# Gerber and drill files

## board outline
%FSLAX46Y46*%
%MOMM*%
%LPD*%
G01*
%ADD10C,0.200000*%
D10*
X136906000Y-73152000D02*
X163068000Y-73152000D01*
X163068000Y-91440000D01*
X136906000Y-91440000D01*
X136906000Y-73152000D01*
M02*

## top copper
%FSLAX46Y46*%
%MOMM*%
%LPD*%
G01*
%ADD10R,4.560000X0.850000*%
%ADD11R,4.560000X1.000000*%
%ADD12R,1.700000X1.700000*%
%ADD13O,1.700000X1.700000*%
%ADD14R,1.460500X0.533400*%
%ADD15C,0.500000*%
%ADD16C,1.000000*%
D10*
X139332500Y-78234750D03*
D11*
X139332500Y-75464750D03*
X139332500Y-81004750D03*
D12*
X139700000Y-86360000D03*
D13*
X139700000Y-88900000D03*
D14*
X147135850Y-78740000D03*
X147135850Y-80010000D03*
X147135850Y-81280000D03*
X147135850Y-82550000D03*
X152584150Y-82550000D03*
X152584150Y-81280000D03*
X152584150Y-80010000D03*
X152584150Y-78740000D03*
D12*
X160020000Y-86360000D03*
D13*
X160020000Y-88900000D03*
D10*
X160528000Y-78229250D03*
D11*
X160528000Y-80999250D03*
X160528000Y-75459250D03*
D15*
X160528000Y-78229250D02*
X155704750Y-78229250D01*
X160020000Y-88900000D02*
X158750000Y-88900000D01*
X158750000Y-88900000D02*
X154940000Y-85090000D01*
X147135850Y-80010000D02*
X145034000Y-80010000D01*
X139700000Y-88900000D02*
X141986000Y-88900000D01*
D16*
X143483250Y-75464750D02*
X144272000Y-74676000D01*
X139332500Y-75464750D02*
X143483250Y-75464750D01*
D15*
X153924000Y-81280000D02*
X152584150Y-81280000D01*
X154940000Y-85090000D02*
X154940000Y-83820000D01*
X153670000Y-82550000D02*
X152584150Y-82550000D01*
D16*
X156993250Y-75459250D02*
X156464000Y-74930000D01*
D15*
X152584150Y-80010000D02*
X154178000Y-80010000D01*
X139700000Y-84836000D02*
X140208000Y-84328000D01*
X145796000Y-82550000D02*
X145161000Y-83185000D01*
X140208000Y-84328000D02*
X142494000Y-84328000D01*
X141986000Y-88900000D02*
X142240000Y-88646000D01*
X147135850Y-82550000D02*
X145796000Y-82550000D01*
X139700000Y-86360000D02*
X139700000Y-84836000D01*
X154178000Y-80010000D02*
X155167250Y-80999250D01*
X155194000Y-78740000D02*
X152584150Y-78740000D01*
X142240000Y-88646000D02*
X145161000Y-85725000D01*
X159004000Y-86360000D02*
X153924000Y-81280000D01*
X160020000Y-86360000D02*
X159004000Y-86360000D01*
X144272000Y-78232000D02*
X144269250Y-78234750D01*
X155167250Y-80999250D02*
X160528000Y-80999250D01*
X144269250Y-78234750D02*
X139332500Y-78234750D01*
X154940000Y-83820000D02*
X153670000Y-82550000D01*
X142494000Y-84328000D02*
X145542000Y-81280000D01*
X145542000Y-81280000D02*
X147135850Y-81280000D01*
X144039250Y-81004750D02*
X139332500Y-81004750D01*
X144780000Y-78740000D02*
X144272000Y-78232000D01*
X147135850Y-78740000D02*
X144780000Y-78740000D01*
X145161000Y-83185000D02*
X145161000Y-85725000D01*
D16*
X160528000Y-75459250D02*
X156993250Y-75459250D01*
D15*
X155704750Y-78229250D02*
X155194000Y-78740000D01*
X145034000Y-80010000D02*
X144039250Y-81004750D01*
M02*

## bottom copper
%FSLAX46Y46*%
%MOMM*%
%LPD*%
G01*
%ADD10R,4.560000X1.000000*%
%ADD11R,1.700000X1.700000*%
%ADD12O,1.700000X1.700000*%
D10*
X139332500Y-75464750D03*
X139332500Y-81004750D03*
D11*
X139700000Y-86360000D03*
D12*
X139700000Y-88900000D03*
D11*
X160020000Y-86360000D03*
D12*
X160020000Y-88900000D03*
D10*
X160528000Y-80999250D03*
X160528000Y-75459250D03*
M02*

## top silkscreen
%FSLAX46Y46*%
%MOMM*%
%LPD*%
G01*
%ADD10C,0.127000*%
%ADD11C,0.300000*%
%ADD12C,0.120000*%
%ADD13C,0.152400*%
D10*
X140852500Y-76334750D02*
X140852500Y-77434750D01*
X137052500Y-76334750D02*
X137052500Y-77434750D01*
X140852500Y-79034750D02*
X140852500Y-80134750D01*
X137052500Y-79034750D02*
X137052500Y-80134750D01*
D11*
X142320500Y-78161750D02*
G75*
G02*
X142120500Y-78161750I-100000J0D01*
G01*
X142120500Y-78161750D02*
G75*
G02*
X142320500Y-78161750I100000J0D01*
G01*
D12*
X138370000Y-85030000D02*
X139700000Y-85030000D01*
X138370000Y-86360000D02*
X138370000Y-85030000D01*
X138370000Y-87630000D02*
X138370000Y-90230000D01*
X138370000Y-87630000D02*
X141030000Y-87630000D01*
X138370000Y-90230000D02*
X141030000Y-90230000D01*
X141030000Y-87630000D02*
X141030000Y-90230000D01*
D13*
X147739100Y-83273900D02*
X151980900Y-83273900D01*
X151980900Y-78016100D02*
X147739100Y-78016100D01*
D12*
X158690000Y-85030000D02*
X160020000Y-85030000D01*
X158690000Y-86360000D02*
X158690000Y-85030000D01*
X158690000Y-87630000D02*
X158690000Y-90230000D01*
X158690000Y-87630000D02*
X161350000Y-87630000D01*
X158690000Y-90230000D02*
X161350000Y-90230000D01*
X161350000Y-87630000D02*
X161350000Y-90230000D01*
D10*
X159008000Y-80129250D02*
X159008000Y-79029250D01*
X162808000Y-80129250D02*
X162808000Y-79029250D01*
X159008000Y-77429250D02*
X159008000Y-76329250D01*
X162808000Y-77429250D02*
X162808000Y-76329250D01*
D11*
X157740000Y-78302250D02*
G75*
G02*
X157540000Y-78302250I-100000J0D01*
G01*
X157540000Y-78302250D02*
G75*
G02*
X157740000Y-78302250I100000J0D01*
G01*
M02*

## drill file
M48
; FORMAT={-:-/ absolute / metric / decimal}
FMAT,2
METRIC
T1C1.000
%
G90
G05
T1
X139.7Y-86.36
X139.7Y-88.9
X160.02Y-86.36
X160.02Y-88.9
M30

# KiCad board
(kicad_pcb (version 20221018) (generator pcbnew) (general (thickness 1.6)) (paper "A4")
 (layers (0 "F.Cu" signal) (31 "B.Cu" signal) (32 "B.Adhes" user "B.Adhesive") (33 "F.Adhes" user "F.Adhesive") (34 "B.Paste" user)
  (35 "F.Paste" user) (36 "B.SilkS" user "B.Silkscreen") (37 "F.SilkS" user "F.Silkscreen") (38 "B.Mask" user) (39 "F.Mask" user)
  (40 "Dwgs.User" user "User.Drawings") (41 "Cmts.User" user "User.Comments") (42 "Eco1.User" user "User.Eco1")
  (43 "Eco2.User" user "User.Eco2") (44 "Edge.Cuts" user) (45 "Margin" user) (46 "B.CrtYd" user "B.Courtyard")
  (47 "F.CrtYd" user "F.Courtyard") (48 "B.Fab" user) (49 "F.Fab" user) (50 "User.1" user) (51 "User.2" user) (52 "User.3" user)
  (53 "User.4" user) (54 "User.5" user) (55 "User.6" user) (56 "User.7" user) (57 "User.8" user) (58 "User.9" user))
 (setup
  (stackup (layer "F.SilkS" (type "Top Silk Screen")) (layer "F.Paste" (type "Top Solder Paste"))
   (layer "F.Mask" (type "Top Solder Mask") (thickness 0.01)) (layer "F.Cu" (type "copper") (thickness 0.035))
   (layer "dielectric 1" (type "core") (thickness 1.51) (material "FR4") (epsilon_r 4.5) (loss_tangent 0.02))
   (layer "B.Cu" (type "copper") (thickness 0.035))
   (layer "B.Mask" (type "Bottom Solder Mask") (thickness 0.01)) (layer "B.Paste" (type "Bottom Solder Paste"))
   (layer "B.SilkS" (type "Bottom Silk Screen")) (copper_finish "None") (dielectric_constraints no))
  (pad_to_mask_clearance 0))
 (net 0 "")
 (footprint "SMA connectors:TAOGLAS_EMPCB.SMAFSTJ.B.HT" (layer "F.Cu") (at 139.3325 78.23475 -90)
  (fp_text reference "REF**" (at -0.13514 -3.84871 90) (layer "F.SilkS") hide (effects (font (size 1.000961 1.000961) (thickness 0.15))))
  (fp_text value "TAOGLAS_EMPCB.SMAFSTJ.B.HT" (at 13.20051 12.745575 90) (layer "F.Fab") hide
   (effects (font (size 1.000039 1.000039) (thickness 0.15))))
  (fp_line (start -1.9 -1.52) (end -0.8 -1.52) (stroke (width 0.127) (type solid)) (layer "F.SilkS"))
  (fp_line (start -1.9 2.28) (end -0.8 2.28) (stroke (width 0.127) (type solid)) (layer "F.SilkS"))
  (fp_line (start 0.8 -1.52) (end 1.9 -1.52) (stroke (width 0.127) (type solid)) (layer "F.SilkS"))
  (fp_line (start 0.8 2.28) (end 1.9 2.28) (stroke (width 0.127) (type solid)) (layer "F.SilkS"))
  (fp_circle (center -0.073 -2.888) (end 0.027 -2.888) (stroke (width 0.3) (type solid)) (fill none) (layer "F.SilkS"))
  (pad "1" smd rect (at 0 0 270) (size 0.85 4.56) (layers "F.Cu" "F.Paste" "F.Mask") (solder_mask_margin 0.102))
  (pad "SH1" smd rect (at -2.77 0 270) (size 1 4.56) (layers "F.Cu" "F.Paste" "F.Mask") (solder_mask_margin 0.102))
  (pad "SH2" smd rect (at 2.77 0 270) (size 1 4.56) (layers "F.Cu" "F.Paste" "F.Mask") (solder_mask_margin 0.102))
  (pad "SH3" smd rect (at -2.77 0 270) (size 1 4.56) (layers "B.Cu" "B.Paste" "B.Mask") (solder_mask_margin 0.102))
  (pad "SH4" smd rect (at 2.77 0 270) (size 1 4.56) (layers "B.Cu" "B.Paste" "B.Mask") (solder_mask_margin 0.102)))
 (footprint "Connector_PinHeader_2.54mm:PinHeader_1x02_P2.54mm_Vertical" (layer "F.Cu") (at 139.7 86.36)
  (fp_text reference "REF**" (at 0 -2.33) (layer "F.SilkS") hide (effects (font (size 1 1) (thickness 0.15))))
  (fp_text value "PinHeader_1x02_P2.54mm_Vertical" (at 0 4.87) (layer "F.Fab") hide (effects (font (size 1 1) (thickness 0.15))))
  (fp_line (start -1.33 -1.33) (end 0 -1.33) (stroke (width 0.12) (type solid)) (layer "F.SilkS"))
  (fp_line (start -1.33 0) (end -1.33 -1.33) (stroke (width 0.12) (type solid)) (layer "F.SilkS"))
  (fp_line (start -1.33 1.27) (end -1.33 3.87) (stroke (width 0.12) (type solid)) (layer "F.SilkS"))
  (fp_line (start -1.33 1.27) (end 1.33 1.27) (stroke (width 0.12) (type solid)) (layer "F.SilkS"))
  (fp_line (start -1.33 3.87) (end 1.33 3.87) (stroke (width 0.12) (type solid)) (layer "F.SilkS"))
  (fp_line (start 1.33 1.27) (end 1.33 3.87) (stroke (width 0.12) (type solid)) (layer "F.SilkS"))
  (pad "1" thru_hole rect (at 0 0) (size 1.7 1.7) (drill 1) (layers "*.Cu" "*.Mask"))
  (pad "2" thru_hole oval (at 0 2.54) (size 1.7 1.7) (drill 1) (layers "*.Cu" "*.Mask")))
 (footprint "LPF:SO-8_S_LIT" (layer "F.Cu") (at 149.86 80.645)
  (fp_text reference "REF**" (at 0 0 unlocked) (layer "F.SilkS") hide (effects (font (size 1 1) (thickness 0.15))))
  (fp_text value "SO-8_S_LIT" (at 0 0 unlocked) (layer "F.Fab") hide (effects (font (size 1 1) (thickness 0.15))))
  (fp_line (start -2.1209 2.6289) (end 2.1209 2.6289) (stroke (width 0.1524) (type solid)) (layer "F.SilkS"))
  (fp_line (start 2.1209 -2.6289) (end -2.1209 -2.6289) (stroke (width 0.1524) (type solid)) (layer "F.SilkS"))
  (pad "1" smd rect (at -2.72415 -1.905) (size 1.4605 0.5334) (layers "F.Cu" "F.Paste" "F.Mask"))
  (pad "2" smd rect (at -2.72415 -0.635) (size 1.4605 0.5334) (layers "F.Cu" "F.Paste" "F.Mask"))
  (pad "3" smd rect (at -2.72415 0.635) (size 1.4605 0.5334) (layers "F.Cu" "F.Paste" "F.Mask"))
  (pad "4" smd rect (at -2.72415 1.905) (size 1.4605 0.5334) (layers "F.Cu" "F.Paste" "F.Mask"))
  (pad "5" smd rect (at 2.72415 1.905) (size 1.4605 0.5334) (layers "F.Cu" "F.Paste" "F.Mask"))
  (pad "6" smd rect (at 2.72415 0.635) (size 1.4605 0.5334) (layers "F.Cu" "F.Paste" "F.Mask"))
  (pad "7" smd rect (at 2.72415 -0.635) (size 1.4605 0.5334) (layers "F.Cu" "F.Paste" "F.Mask"))
  (pad "8" smd rect (at 2.72415 -1.905) (size 1.4605 0.5334) (layers "F.Cu" "F.Paste" "F.Mask")))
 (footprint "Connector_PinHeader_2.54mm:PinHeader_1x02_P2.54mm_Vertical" (layer "F.Cu") (at 160.02 86.36)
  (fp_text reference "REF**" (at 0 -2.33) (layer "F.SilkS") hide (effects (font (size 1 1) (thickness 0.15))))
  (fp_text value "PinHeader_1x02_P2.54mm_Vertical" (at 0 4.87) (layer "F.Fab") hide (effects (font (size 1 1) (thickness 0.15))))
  (fp_line (start -1.33 -1.33) (end 0 -1.33) (stroke (width 0.12) (type solid)) (layer "F.SilkS"))
  (fp_line (start -1.33 0) (end -1.33 -1.33) (stroke (width 0.12) (type solid)) (layer "F.SilkS"))
  (fp_line (start -1.33 1.27) (end -1.33 3.87) (stroke (width 0.12) (type solid)) (layer "F.SilkS"))
  (fp_line (start -1.33 1.27) (end 1.33 1.27) (stroke (width 0.12) (type solid)) (layer "F.SilkS"))
  (fp_line (start -1.33 3.87) (end 1.33 3.87) (stroke (width 0.12) (type solid)) (layer "F.SilkS"))
  (fp_line (start 1.33 1.27) (end 1.33 3.87) (stroke (width 0.12) (type solid)) (layer "F.SilkS"))
  (pad "1" thru_hole rect (at 0 0) (size 1.7 1.7) (drill 1) (layers "*.Cu" "*.Mask"))
  (pad "2" thru_hole oval (at 0 2.54) (size 1.7 1.7) (drill 1) (layers "*.Cu" "*.Mask")))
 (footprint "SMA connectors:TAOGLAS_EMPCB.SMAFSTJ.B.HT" (layer "F.Cu") (at 160.528 78.22925 90)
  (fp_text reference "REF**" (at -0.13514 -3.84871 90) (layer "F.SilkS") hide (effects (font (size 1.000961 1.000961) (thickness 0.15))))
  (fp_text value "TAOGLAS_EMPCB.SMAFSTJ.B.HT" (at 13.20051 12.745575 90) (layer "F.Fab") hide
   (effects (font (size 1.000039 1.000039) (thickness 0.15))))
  (fp_line (start -1.9 -1.52) (end -0.8 -1.52) (stroke (width 0.127) (type solid)) (layer "F.SilkS"))
  (fp_line (start -1.9 2.28) (end -0.8 2.28) (stroke (width 0.127) (type solid)) (layer "F.SilkS"))
  (fp_line (start 0.8 -1.52) (end 1.9 -1.52) (stroke (width 0.127) (type solid)) (layer "F.SilkS"))
  (fp_line (start 0.8 2.28) (end 1.9 2.28) (stroke (width 0.127) (type solid)) (layer "F.SilkS"))
  (fp_circle (center -0.073 -2.888) (end 0.027 -2.888) (stroke (width 0.3) (type solid)) (fill none) (layer "F.SilkS"))
  (pad "1" smd rect (at 0 0 90) (size 0.85 4.56) (layers "F.Cu" "F.Paste" "F.Mask") (solder_mask_margin 0.102))
  (pad "SH1" smd rect (at -2.77 0 90) (size 1 4.56) (layers "F.Cu" "F.Paste" "F.Mask") (solder_mask_margin 0.102))
  (pad "SH2" smd rect (at 2.77 0 90) (size 1 4.56) (layers "F.Cu" "F.Paste" "F.Mask") (solder_mask_margin 0.102))
  (pad "SH3" smd rect (at -2.77 0 90) (size 1 4.56) (layers "B.Cu" "B.Paste" "B.Mask") (solder_mask_margin 0.102))
  (pad "SH4" smd rect (at 2.77 0 90) (size 1 4.56) (layers "B.Cu" "B.Paste" "B.Mask") (solder_mask_margin 0.102)))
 (gr_rect (start 136.906 73.152) (end 163.068 91.44) (stroke (width 0.2) (type default)) (fill none) (layer "Edge.Cuts"))
 (segment (start 160.528 78.22925) (end 155.70475 78.22925) (width 0.5) (layer "F.Cu") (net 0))
 (segment (start 160.02 88.9) (end 158.75 88.9) (width 0.5) (layer "F.Cu") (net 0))
 (segment (start 158.75 88.9) (end 154.94 85.09) (width 0.5) (layer "F.Cu") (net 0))
 (segment (start 147.13585 80.01) (end 145.034 80.01) (width 0.5) (layer "F.Cu") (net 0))
 (segment (start 139.7 88.9) (end 141.986 88.9) (width 0.5) (layer "F.Cu") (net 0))
 (segment (start 143.48325 75.46475) (end 144.272 74.676) (width 1) (layer "F.Cu") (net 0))
 (segment (start 139.3325 75.46475) (end 143.48325 75.46475) (width 1) (layer "F.Cu") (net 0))
 (segment (start 153.924 81.28) (end 152.58415 81.28) (width 0.5) (layer "F.Cu") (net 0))
 (segment (start 154.94 85.09) (end 154.94 83.82) (width 0.5) (layer "F.Cu") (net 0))
 (segment (start 153.67 82.55) (end 152.58415 82.55) (width 0.5) (layer "F.Cu") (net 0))
 (segment (start 156.99325 75.45925) (end 156.464 74.93) (width 1) (layer "F.Cu") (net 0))
 (segment (start 152.58415 80.01) (end 154.178 80.01) (width 0.5) (layer "F.Cu") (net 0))
 (segment (start 139.7 84.836) (end 140.208 84.328) (width 0.5) (layer "F.Cu") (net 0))
 (segment (start 145.796 82.55) (end 145.161 83.185) (width 0.5) (layer "F.Cu") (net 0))
 (segment (start 140.208 84.328) (end 142.494 84.328) (width 0.5) (layer "F.Cu") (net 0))
 (segment (start 141.986 88.9) (end 142.24 88.646) (width 0.5) (layer "F.Cu") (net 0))
 (segment (start 147.13585 82.55) (end 145.796 82.55) (width 0.5) (layer "F.Cu") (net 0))
 (segment (start 139.7 86.36) (end 139.7 84.836) (width 0.5) (layer "F.Cu") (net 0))
 (segment (start 154.178 80.01) (end 155.16725 80.99925) (width 0.5) (layer "F.Cu") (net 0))
 (segment (start 155.194 78.74) (end 152.58415 78.74) (width 0.5) (layer "F.Cu") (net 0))
 (segment (start 142.24 88.646) (end 145.161 85.725) (width 0.5) (layer "F.Cu") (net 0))
 (segment (start 159.004 86.36) (end 153.924 81.28) (width 0.5) (layer "F.Cu") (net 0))
 (segment (start 160.02 86.36) (end 159.004 86.36) (width 0.5) (layer "F.Cu") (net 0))
 (segment (start 144.272 78.232) (end 144.26925 78.23475) (width 0.5) (layer "F.Cu") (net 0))
 (segment (start 155.16725 80.99925) (end 160.528 80.99925) (width 0.5) (layer "F.Cu") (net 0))
 (segment (start 144.26925 78.23475) (end 139.3325 78.23475) (width 0.5) (layer "F.Cu") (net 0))
 (segment (start 154.94 83.82) (end 153.67 82.55) (width 0.5) (layer "F.Cu") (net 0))
 (segment (start 142.494 84.328) (end 145.542 81.28) (width 0.5) (layer "F.Cu") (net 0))
 (segment (start 145.542 81.28) (end 147.13585 81.28) (width 0.5) (layer "F.Cu") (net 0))
 (segment (start 144.03925 81.00475) (end 139.3325 81.00475) (width 0.5) (layer "F.Cu") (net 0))
 (segment (start 144.78 78.74) (end 144.272 78.232) (width 0.5) (layer "F.Cu") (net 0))
 (segment (start 147.13585 78.74) (end 144.78 78.74) (width 0.5) (layer "F.Cu") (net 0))
 (segment (start 145.161 83.185) (end 145.161 85.725) (width 0.5) (layer "F.Cu") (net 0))
 (segment (start 160.528 75.45925) (end 156.99325 75.45925) (width 1) (layer "F.Cu") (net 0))
 (segment (start 155.70475 78.22925) (end 155.194 78.74) (width 0.5) (layer "F.Cu") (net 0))
 (segment (start 145.034 80.01) (end 144.03925 81.00475) (width 0.5) (layer "F.Cu") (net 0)))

